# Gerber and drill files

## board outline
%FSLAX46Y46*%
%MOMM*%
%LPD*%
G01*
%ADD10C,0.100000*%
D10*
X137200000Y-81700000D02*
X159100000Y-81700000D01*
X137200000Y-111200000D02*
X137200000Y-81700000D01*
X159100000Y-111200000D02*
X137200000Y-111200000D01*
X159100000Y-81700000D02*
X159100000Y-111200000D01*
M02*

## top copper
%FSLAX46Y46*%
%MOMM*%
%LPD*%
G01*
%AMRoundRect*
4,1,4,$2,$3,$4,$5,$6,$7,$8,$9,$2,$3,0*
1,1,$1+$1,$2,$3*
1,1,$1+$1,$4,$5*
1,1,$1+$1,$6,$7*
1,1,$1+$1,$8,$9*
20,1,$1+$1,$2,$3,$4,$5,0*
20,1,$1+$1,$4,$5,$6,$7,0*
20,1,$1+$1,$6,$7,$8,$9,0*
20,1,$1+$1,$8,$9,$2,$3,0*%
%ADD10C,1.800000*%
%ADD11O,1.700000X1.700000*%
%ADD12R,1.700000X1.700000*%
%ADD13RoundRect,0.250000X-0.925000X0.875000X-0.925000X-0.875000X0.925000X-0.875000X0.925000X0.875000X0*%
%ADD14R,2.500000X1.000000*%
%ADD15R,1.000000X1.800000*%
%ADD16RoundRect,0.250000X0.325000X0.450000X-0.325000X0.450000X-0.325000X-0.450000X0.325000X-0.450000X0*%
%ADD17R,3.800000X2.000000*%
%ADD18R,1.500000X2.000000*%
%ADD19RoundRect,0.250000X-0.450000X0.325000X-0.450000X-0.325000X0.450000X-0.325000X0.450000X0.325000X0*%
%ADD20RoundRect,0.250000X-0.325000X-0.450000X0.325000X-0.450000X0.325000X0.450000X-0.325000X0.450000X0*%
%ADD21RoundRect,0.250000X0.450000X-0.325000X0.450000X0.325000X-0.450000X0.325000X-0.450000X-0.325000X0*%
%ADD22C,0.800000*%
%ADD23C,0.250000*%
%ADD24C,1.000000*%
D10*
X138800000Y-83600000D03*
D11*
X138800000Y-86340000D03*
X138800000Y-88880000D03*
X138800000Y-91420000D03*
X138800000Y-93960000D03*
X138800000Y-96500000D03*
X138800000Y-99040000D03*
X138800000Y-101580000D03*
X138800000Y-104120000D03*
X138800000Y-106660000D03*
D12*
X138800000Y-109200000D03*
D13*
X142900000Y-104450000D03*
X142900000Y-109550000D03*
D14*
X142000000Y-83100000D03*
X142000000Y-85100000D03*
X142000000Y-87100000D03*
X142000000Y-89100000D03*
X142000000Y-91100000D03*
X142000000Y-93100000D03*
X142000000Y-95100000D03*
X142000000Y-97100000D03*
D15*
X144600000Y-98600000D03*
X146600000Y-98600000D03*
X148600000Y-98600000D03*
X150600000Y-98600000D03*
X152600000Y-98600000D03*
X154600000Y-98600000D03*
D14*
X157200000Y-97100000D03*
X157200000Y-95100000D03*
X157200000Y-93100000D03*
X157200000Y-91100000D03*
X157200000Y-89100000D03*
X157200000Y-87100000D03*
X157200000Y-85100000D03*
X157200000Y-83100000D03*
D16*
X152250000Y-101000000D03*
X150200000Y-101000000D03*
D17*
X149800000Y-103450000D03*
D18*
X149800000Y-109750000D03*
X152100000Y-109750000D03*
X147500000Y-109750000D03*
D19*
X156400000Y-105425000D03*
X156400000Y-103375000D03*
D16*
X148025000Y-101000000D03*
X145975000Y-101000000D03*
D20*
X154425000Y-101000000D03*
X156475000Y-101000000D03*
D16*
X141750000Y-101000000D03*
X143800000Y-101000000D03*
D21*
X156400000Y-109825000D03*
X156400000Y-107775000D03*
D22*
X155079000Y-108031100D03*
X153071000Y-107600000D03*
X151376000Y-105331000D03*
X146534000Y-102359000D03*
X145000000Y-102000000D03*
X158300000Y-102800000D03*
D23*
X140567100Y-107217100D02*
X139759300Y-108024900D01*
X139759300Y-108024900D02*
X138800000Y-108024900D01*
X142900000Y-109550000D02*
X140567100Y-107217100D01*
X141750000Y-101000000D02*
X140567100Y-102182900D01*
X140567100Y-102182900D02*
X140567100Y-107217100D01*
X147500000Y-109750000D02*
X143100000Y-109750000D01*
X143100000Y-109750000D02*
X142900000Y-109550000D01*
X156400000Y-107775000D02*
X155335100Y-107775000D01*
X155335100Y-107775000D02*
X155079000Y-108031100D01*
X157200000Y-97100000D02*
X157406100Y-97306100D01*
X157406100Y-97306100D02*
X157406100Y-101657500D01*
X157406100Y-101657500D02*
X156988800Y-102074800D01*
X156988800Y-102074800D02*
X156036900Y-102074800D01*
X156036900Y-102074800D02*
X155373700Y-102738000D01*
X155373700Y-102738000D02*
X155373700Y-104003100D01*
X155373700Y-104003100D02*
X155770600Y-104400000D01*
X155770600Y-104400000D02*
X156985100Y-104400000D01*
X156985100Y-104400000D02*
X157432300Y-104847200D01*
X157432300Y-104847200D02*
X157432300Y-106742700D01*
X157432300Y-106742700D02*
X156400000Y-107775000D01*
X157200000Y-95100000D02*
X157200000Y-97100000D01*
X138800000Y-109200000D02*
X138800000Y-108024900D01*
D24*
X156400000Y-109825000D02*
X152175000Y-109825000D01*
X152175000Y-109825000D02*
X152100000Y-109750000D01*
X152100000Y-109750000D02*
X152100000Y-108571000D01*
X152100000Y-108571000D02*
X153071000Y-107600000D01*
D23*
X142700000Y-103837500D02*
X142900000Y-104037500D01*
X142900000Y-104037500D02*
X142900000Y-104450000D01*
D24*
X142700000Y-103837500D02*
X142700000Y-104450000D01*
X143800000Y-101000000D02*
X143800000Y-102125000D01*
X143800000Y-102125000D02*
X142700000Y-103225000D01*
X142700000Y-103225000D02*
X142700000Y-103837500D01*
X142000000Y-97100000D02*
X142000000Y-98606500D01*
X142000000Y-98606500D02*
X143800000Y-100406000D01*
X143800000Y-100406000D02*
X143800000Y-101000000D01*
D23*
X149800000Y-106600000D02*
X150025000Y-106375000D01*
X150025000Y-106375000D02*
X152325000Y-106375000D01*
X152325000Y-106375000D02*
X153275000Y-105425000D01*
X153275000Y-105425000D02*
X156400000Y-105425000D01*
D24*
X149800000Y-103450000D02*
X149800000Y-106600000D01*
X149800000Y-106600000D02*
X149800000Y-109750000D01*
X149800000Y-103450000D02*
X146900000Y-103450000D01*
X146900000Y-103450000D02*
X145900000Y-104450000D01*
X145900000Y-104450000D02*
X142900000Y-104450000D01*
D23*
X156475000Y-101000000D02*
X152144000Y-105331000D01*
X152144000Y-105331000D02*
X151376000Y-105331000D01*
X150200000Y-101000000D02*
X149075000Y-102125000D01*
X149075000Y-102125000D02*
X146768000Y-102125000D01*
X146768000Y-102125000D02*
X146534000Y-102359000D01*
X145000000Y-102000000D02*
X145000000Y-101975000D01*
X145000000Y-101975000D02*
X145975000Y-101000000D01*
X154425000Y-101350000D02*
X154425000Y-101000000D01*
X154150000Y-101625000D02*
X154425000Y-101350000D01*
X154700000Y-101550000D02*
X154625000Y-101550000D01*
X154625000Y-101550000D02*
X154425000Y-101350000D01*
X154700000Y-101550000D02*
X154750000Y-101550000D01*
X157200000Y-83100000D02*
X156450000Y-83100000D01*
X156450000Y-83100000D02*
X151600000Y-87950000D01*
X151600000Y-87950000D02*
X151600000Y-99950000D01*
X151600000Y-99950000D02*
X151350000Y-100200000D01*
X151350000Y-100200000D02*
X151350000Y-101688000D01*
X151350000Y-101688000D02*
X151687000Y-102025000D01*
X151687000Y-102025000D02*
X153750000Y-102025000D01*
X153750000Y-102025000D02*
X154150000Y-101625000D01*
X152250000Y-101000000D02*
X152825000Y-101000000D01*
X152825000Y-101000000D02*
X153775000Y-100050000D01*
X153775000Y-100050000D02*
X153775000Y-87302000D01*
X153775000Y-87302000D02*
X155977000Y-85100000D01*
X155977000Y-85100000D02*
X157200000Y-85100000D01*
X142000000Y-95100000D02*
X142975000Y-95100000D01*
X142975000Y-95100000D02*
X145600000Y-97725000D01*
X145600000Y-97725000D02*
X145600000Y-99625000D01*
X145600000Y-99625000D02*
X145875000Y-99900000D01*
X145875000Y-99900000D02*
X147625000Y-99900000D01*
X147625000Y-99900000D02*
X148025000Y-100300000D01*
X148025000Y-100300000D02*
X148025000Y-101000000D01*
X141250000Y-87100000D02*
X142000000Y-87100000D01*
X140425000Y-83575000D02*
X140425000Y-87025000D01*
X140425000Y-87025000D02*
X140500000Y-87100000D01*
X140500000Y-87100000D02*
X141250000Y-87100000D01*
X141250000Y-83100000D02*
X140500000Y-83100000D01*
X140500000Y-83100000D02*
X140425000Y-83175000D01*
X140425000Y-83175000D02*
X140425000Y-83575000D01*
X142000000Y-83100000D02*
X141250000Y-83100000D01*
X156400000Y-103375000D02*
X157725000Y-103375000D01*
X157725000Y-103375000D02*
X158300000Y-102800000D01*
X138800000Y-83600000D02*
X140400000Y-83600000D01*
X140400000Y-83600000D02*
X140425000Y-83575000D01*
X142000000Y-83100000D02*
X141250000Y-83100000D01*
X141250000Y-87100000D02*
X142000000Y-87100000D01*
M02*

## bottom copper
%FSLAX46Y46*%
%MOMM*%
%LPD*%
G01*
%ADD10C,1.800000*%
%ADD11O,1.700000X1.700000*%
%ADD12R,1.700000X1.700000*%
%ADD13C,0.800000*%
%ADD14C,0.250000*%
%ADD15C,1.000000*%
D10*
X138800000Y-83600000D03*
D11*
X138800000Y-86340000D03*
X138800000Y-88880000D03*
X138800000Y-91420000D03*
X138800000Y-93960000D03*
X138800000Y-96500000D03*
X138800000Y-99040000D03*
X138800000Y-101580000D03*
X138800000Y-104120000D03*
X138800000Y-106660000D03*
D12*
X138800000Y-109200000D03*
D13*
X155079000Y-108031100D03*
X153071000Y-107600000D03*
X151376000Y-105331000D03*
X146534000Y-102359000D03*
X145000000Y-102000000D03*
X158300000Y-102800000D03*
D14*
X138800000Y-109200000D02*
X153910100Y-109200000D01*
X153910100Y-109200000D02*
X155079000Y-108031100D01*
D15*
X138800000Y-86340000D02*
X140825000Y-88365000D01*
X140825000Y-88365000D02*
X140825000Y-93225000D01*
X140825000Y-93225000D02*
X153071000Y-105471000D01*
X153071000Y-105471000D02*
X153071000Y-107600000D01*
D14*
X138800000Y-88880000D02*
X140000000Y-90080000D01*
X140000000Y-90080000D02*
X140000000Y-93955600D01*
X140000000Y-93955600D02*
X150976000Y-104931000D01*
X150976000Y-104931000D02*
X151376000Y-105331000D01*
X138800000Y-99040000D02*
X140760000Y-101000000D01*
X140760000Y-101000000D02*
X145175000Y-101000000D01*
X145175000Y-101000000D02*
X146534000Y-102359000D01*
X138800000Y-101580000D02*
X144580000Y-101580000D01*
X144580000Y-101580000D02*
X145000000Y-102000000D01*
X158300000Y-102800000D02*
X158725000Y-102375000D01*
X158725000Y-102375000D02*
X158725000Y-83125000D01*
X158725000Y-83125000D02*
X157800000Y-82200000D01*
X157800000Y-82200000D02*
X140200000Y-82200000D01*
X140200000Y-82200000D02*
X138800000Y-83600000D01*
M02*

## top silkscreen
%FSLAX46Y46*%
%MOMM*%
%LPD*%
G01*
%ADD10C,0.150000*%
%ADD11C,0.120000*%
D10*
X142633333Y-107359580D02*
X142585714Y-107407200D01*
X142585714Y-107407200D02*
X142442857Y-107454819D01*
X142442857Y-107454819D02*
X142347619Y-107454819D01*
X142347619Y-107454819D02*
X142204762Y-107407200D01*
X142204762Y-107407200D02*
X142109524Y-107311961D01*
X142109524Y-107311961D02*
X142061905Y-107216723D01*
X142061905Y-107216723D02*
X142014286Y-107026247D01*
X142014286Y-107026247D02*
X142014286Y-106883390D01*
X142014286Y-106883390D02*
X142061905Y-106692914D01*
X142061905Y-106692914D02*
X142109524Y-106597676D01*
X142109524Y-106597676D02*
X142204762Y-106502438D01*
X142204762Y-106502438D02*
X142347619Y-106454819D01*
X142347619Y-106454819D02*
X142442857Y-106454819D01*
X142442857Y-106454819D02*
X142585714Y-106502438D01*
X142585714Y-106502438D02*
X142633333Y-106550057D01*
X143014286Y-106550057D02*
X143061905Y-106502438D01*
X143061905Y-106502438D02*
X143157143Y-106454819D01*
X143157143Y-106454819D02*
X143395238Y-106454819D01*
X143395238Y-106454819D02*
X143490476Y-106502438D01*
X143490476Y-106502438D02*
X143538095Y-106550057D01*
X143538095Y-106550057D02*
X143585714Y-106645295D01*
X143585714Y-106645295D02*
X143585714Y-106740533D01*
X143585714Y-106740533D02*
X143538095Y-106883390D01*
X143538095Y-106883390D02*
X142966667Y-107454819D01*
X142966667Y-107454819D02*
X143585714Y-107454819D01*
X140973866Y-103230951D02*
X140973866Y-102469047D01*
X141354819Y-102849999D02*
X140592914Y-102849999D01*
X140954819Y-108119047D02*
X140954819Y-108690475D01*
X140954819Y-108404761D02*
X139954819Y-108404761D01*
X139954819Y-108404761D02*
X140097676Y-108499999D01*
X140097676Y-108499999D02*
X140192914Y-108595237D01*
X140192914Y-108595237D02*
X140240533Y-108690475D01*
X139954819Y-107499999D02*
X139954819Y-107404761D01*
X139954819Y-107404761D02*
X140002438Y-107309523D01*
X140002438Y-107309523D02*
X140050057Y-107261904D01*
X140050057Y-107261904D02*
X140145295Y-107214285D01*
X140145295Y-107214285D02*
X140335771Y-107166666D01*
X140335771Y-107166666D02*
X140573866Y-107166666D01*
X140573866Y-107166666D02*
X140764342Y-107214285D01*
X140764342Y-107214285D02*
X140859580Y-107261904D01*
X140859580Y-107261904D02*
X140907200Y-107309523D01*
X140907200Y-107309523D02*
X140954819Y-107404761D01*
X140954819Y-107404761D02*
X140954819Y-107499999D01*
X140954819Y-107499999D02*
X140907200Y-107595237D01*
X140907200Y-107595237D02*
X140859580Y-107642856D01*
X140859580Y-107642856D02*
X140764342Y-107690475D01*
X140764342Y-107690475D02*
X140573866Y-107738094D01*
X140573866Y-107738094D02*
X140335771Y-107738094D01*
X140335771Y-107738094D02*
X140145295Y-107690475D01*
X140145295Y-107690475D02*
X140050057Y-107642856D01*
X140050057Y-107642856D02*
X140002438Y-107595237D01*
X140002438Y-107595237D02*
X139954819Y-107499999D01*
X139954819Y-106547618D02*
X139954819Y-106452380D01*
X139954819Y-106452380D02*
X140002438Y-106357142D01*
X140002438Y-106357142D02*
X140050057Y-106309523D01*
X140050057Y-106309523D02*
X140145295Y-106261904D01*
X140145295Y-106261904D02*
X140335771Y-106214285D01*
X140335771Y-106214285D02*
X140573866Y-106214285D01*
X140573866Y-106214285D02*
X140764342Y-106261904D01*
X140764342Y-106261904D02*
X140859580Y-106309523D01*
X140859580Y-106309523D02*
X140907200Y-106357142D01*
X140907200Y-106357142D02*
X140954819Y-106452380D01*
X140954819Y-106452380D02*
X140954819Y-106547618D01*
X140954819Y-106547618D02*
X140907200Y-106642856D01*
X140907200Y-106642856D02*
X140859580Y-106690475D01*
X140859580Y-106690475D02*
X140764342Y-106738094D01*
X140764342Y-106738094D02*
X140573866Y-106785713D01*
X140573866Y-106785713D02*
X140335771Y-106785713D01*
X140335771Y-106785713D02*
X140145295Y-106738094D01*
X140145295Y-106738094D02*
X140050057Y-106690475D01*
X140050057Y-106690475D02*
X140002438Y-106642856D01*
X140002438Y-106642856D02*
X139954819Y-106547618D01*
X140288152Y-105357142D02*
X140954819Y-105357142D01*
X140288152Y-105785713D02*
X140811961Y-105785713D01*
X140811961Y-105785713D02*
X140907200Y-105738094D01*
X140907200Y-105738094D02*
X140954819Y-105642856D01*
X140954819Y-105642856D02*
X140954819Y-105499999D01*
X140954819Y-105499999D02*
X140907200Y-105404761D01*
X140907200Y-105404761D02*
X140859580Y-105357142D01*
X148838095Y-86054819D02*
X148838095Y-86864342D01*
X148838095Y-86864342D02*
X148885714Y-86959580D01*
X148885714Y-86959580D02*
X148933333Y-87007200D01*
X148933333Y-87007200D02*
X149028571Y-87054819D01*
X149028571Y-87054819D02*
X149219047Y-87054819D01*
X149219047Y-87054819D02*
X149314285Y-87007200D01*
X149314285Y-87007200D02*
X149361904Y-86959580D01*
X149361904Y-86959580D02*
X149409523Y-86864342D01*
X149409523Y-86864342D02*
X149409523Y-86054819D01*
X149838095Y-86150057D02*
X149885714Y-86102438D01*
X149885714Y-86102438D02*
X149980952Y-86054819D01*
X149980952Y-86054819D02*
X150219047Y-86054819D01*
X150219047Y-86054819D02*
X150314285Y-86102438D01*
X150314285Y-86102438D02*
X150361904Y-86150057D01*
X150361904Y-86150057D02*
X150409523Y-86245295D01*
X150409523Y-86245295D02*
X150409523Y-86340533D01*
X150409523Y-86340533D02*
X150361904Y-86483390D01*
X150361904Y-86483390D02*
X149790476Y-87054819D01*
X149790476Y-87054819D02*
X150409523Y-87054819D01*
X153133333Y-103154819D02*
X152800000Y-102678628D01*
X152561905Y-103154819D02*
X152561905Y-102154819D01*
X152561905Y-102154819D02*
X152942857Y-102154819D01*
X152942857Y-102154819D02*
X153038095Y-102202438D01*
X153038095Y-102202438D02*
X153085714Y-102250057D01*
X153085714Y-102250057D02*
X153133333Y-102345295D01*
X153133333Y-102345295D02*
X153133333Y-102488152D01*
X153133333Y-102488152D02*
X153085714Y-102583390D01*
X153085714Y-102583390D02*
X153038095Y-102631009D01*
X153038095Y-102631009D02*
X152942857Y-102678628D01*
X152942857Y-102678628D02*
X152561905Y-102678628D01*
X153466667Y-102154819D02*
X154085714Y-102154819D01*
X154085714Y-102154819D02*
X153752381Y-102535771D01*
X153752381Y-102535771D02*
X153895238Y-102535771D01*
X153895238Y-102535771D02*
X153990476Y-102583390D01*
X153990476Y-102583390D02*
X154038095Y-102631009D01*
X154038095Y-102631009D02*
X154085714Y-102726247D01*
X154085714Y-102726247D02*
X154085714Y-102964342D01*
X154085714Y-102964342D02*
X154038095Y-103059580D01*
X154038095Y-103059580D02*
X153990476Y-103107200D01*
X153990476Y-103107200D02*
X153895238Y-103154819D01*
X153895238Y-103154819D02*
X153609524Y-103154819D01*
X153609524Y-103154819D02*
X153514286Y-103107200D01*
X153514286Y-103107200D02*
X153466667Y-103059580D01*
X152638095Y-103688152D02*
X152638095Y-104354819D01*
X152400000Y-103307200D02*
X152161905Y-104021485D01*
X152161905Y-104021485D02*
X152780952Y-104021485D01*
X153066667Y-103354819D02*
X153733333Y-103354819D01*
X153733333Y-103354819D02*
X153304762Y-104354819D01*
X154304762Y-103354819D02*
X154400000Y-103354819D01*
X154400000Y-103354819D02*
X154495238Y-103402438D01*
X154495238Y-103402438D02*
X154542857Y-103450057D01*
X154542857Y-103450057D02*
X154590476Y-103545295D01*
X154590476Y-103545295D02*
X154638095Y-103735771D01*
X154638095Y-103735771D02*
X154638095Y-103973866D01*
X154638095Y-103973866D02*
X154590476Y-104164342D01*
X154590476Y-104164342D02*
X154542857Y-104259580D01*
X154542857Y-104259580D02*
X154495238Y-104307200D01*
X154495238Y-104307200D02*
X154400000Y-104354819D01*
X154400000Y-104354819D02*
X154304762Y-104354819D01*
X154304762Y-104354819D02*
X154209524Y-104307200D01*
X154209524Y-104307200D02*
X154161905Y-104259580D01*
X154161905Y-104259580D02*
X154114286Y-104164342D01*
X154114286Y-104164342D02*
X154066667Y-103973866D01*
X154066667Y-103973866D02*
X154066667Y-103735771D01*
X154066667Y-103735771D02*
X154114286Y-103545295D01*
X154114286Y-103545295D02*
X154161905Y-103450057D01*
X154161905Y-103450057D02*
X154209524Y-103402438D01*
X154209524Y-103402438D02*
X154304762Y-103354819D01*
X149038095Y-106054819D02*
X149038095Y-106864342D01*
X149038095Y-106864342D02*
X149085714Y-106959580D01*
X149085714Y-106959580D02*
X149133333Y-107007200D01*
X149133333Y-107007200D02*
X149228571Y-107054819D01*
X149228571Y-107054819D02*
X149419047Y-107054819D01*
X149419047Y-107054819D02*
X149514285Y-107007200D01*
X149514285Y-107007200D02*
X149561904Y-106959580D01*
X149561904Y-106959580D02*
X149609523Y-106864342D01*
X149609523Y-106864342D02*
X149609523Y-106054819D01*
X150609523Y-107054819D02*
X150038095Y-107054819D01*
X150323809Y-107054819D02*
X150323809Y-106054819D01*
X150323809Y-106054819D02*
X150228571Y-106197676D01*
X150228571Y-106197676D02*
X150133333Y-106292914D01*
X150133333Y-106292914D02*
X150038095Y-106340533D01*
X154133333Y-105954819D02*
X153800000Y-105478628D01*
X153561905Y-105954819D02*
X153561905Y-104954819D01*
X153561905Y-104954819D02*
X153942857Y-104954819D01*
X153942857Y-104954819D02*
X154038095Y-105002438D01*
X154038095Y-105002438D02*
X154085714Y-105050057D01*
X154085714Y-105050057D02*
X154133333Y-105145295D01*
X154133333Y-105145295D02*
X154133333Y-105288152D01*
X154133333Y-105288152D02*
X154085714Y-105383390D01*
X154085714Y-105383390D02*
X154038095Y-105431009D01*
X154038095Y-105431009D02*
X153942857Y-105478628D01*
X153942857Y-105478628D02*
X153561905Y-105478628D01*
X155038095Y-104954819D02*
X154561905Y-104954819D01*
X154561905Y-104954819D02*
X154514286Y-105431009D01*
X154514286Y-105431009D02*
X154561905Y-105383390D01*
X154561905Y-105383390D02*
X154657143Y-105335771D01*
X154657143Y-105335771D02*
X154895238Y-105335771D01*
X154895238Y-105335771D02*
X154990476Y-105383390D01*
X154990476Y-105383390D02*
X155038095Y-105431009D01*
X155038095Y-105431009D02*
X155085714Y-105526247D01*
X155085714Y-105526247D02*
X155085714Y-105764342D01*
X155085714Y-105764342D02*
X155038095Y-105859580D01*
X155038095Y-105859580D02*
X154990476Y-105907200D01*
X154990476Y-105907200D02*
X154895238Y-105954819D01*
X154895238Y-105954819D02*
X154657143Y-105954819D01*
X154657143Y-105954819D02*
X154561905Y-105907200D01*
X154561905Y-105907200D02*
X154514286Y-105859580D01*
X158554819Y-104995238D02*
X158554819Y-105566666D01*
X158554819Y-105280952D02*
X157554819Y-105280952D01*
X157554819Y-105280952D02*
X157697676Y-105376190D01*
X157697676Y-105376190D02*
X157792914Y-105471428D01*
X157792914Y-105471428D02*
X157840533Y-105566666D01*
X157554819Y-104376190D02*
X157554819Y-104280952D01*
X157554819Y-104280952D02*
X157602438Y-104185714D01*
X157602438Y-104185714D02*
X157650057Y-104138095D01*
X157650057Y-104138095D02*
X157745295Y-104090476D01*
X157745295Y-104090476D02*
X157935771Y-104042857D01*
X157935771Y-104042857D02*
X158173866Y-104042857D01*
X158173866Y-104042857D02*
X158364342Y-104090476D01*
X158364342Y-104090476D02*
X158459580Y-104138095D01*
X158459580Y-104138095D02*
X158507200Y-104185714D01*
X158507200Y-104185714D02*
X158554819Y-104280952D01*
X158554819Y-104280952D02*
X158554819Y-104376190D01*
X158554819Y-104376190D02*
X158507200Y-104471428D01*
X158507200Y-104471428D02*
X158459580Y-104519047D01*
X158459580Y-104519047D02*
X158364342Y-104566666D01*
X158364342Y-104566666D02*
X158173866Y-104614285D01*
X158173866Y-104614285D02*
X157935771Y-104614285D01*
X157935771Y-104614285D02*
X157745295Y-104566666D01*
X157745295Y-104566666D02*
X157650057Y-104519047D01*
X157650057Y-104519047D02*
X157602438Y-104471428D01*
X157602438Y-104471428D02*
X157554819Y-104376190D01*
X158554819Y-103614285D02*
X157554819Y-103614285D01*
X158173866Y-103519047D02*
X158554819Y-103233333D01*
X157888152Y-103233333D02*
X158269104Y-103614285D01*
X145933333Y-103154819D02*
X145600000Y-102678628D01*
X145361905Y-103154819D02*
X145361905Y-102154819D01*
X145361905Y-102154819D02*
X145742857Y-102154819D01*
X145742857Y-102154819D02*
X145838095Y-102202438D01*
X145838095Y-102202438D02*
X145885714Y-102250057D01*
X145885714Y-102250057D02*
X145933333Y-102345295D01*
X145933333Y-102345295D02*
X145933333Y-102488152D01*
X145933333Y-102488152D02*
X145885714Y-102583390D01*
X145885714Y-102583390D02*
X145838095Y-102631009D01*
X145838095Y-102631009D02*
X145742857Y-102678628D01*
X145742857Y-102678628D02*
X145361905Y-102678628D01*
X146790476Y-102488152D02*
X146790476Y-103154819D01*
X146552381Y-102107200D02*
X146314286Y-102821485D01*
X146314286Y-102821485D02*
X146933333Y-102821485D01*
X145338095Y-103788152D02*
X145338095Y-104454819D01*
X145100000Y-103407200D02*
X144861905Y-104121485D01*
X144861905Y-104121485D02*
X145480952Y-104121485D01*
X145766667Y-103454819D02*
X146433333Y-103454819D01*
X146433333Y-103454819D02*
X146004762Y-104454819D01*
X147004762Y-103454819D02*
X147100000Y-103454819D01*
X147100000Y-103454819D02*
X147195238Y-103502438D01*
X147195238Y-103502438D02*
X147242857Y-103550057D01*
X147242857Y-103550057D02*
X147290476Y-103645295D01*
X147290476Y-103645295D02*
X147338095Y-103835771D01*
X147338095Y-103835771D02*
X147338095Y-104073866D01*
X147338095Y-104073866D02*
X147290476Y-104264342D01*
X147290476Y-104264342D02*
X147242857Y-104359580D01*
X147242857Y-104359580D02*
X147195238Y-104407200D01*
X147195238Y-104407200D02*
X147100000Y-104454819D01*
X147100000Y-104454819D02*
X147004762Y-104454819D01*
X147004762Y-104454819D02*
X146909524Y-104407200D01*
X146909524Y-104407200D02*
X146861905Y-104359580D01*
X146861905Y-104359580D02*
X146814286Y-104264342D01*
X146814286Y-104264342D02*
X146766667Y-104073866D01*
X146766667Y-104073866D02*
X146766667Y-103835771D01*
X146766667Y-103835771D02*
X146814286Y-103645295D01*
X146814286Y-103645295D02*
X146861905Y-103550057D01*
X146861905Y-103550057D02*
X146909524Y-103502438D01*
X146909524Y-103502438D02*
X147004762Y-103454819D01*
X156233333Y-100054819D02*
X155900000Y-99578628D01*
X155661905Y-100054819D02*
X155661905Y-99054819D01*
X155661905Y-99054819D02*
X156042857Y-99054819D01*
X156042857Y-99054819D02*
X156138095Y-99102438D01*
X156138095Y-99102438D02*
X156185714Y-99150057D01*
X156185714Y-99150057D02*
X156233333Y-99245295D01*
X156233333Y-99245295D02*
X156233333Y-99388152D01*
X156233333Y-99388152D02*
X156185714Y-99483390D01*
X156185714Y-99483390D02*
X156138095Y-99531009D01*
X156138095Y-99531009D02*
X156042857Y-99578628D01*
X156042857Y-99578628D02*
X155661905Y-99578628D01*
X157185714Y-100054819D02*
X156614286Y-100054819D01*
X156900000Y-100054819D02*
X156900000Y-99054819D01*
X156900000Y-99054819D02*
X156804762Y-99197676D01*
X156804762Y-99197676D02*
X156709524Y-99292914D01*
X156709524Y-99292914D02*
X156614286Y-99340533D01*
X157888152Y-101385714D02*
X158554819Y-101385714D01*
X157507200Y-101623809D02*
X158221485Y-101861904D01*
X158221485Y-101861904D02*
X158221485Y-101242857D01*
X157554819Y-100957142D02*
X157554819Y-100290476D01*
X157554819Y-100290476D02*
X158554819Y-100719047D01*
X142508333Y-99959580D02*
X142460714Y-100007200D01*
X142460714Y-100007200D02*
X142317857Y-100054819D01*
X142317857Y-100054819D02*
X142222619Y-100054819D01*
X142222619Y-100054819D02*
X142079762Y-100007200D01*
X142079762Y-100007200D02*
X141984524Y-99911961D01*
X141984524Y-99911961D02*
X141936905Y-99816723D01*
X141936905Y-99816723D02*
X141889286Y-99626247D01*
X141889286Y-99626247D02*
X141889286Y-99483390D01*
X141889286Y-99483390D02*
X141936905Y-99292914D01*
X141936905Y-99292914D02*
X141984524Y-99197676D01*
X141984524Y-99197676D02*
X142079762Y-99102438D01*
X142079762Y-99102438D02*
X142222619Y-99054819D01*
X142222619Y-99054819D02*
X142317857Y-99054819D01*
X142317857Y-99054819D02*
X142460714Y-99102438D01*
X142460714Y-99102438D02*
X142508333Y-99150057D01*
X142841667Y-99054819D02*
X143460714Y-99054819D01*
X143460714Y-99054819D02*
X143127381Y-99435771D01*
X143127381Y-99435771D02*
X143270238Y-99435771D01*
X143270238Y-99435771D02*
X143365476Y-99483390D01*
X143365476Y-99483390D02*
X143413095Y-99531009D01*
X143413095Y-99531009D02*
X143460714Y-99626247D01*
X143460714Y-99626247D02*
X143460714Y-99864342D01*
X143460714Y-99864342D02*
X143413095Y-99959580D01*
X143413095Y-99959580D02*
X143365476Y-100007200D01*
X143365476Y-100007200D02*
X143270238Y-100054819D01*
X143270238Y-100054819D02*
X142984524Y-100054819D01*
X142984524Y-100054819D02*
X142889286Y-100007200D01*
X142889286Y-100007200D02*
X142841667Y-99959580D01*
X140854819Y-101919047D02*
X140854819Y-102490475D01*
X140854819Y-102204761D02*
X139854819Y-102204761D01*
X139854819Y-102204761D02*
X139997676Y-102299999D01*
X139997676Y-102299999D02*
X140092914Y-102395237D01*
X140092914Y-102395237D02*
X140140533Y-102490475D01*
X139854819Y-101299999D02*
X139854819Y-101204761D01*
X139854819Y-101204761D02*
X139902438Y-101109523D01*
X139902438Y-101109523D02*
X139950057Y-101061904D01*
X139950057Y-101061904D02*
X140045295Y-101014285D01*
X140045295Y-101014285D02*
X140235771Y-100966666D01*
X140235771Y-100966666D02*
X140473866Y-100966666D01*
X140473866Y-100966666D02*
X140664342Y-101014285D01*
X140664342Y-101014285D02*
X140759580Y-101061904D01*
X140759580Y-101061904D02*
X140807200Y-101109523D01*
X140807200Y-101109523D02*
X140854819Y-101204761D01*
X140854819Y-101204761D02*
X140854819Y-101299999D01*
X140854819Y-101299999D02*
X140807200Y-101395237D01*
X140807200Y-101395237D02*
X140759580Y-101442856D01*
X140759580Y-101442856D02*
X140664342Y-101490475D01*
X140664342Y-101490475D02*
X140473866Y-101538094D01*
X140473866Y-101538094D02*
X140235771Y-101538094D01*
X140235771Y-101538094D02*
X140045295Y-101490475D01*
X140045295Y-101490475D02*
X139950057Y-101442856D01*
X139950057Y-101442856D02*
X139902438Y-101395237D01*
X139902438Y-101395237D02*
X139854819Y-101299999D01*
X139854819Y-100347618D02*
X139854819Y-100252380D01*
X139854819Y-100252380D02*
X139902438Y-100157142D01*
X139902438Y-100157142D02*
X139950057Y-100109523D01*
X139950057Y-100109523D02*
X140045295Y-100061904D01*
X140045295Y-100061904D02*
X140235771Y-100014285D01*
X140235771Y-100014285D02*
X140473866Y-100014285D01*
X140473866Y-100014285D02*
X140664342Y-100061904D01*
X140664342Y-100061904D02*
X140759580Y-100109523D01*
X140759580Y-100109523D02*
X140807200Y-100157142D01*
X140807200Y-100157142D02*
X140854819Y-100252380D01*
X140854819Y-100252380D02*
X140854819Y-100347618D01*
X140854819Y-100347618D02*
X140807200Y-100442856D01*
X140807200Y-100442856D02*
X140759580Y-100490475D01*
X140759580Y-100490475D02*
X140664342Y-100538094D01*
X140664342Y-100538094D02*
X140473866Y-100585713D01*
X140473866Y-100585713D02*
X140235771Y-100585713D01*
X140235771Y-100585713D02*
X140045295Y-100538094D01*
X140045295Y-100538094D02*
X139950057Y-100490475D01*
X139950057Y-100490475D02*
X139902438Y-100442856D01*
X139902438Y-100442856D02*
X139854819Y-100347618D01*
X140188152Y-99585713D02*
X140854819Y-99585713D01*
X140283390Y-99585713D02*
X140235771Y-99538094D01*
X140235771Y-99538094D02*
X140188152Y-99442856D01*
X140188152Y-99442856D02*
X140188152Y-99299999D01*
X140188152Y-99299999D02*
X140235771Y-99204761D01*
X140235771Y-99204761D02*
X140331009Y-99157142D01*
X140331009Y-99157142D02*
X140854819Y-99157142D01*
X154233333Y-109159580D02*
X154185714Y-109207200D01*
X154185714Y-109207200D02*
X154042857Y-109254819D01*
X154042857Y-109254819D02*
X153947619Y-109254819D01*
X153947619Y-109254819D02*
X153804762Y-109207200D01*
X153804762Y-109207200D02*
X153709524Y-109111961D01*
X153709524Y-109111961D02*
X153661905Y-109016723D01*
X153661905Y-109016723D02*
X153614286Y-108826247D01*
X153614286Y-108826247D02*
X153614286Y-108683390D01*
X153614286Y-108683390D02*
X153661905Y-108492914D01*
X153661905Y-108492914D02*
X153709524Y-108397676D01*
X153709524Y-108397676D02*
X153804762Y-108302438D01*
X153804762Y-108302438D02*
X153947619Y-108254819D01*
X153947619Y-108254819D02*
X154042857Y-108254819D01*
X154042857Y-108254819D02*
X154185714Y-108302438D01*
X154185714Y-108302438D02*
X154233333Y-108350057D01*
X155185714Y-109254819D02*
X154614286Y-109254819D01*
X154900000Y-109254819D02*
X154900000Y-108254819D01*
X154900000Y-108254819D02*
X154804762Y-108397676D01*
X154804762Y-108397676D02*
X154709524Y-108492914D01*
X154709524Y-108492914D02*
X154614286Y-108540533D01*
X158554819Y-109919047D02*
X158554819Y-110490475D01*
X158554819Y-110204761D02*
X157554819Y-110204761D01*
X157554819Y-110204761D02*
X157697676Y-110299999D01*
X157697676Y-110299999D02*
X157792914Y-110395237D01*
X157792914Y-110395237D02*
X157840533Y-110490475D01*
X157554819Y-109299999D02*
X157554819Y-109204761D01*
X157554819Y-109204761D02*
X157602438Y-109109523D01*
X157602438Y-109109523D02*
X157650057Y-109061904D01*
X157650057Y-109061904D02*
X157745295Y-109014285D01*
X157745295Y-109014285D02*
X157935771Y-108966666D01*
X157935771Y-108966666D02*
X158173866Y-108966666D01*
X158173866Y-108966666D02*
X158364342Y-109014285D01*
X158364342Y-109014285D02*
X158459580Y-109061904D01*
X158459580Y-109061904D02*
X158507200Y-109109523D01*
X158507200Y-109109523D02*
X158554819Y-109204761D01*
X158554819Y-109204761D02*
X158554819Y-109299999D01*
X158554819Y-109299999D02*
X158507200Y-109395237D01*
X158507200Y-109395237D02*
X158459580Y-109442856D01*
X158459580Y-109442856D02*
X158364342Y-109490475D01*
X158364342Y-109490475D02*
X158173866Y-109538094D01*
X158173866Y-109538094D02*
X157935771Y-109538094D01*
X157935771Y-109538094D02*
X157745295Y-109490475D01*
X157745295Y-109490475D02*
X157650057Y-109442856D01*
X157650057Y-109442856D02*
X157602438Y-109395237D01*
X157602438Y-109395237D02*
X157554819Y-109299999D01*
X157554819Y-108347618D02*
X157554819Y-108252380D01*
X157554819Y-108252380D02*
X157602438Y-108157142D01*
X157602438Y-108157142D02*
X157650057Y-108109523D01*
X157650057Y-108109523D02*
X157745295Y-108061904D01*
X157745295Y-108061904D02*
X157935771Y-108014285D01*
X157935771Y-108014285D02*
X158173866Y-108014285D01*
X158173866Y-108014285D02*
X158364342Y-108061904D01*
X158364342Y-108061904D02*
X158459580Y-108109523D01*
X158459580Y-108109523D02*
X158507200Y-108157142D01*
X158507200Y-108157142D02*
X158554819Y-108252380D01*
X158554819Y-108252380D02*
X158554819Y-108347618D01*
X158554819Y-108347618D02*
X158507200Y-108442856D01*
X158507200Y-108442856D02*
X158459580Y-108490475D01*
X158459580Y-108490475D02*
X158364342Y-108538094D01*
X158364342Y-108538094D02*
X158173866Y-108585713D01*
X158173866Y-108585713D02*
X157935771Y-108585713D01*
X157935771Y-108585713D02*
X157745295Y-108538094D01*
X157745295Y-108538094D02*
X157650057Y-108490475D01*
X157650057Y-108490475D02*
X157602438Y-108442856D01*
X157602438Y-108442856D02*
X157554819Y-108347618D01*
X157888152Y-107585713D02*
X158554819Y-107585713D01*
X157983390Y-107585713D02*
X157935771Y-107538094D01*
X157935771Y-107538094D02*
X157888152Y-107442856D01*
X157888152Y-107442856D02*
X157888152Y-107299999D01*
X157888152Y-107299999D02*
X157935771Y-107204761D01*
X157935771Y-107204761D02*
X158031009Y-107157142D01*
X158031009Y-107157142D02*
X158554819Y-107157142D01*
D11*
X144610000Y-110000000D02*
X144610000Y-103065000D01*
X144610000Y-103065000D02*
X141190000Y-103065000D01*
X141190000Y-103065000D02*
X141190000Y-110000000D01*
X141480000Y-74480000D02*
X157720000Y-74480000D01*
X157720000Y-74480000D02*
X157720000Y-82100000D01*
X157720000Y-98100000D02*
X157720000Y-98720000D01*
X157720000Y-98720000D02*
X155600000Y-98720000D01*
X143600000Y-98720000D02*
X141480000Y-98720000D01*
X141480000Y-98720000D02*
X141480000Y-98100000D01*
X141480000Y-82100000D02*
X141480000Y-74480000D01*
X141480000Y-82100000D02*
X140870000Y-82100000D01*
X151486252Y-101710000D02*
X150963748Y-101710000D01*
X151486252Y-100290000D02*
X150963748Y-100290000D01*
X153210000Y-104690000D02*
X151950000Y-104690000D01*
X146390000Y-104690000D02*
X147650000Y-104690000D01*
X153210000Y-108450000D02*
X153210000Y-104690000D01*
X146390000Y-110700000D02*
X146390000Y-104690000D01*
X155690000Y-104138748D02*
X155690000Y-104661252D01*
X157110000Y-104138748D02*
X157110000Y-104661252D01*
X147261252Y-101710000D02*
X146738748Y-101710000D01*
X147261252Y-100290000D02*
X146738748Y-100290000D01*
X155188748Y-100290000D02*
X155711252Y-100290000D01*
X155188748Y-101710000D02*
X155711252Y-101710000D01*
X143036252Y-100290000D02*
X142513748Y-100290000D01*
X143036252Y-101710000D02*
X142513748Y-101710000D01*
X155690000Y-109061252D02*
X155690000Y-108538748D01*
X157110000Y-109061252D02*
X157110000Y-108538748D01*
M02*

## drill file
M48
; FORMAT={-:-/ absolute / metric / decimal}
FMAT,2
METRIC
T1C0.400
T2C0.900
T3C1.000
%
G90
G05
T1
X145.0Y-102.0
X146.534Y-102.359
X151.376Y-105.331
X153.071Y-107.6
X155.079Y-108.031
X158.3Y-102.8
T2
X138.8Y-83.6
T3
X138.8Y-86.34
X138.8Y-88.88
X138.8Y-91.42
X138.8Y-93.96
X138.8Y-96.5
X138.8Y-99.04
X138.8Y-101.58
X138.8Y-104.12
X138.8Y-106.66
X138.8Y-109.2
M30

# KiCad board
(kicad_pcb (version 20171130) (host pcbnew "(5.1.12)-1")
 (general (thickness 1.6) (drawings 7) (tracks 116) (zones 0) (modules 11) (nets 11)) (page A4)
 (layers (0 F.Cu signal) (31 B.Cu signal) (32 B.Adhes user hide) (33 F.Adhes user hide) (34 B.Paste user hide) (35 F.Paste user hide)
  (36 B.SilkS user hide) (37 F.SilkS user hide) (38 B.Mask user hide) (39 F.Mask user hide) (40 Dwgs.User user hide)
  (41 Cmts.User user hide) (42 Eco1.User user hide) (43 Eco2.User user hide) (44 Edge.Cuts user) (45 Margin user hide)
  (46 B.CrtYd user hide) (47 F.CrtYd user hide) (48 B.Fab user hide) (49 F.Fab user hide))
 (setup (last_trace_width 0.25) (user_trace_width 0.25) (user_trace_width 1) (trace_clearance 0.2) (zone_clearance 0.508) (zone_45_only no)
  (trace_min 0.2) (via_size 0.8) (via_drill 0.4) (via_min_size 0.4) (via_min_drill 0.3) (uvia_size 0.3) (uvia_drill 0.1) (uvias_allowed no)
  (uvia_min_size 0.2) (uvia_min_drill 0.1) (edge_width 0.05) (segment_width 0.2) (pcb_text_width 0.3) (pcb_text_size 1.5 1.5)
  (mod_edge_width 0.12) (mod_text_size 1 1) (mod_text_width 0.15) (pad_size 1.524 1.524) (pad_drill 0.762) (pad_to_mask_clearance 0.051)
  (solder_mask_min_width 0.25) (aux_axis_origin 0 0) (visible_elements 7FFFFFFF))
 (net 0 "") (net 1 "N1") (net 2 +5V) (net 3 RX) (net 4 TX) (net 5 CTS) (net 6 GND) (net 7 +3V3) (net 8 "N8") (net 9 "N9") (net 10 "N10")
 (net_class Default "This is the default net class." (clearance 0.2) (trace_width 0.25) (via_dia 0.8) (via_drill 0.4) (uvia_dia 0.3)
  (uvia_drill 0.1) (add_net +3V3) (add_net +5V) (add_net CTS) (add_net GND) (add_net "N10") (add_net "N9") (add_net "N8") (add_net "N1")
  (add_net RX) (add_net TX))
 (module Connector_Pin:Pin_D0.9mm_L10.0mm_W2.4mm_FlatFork (layer B.Cu) (at 138.8 83.6)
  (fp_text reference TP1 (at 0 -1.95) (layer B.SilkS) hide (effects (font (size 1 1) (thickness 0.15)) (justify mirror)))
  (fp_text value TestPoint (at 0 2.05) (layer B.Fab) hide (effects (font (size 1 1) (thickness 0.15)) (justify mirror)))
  (pad 1 thru_hole circle (at 0 0) (size 1.8 1.8) (drill 0.9) (layers *.Cu *.Mask) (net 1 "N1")))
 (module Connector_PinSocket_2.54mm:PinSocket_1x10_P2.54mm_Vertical (layer B.Cu) (at 138.8 109.2)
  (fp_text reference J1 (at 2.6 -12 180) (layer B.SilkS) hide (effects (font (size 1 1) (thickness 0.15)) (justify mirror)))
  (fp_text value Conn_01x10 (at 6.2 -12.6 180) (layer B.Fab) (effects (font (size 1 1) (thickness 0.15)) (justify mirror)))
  (pad 10 thru_hole oval (at 0 -22.86) (size 1.7 1.7) (drill 1) (layers *.Cu *.Mask) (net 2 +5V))
  (pad 9 thru_hole oval (at 0 -20.32) (size 1.7 1.7) (drill 1) (layers *.Cu *.Mask) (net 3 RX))
  (pad 8 thru_hole oval (at 0 -17.78) (size 1.7 1.7) (drill 1) (layers *.Cu *.Mask))
  (pad 7 thru_hole oval (at 0 -15.24) (size 1.7 1.7) (drill 1) (layers *.Cu *.Mask))
  (pad 6 thru_hole oval (at 0 -12.7) (size 1.7 1.7) (drill 1) (layers *.Cu *.Mask))
  (pad 5 thru_hole oval (at 0 -10.16) (size 1.7 1.7) (drill 1) (layers *.Cu *.Mask) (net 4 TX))
  (pad 4 thru_hole oval (at 0 -7.62) (size 1.7 1.7) (drill 1) (layers *.Cu *.Mask) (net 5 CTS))
  (pad 3 thru_hole oval (at 0 -5.08) (size 1.7 1.7) (drill 1) (layers *.Cu *.Mask))
  (pad 2 thru_hole oval (at 0 -2.54) (size 1.7 1.7) (drill 1) (layers *.Cu *.Mask))
  (pad 1 thru_hole rect (at 0 0) (size 1.7 1.7) (drill 1) (layers *.Cu *.Mask) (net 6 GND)))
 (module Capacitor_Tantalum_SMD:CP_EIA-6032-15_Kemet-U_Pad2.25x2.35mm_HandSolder (layer F.Cu) (at 142.9 107 270)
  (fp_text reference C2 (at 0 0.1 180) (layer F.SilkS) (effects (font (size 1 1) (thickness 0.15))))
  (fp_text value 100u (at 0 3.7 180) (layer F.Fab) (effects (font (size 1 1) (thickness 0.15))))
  (fp_line (start 3 -1.71) (end -3.935 -1.71) (layer F.SilkS) (width 0.12))
  (fp_line (start -3.935 -1.71) (end -3.935 1.71) (layer F.SilkS) (width 0.12))
  (fp_line (start -3.935 1.71) (end 3 1.71) (layer F.SilkS) (width 0.12))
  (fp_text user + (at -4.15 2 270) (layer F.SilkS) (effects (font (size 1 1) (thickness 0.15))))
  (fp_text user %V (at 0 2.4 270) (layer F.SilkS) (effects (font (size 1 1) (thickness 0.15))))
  (pad 1 smd roundrect (at -2.55 0 270) (size 2.25 2.35) (layers F.Cu F.Paste F.Mask) (roundrect_rratio 0.111111) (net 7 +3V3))
  (pad 2 smd roundrect (at 2.55 0 270) (size 2.25 2.35) (layers F.Cu F.Paste F.Mask) (roundrect_rratio 0.111111) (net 6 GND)))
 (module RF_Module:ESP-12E (layer F.Cu) (at 149.6 86.6)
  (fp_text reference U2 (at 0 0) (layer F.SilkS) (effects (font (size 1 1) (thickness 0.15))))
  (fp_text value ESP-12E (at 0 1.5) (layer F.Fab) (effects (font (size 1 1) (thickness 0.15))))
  (fp_line (start -8.12 -12.12) (end 8.12 -12.12) (layer F.SilkS) (width 0.12))
  (fp_line (start 8.12 -12.12) (end 8.12 -4.5) (layer F.SilkS) (width 0.12))
  (fp_line (start 8.12 11.5) (end 8.12 12.12) (layer F.SilkS) (width 0.12))
  (fp_line (start 8.12 12.12) (end 6 12.12) (layer F.SilkS) (width 0.12))
  (fp_line (start -6 12.12) (end -8.12 12.12) (layer F.SilkS) (width 0.12))
  (fp_line (start -8.12 12.12) (end -8.12 11.5) (layer F.SilkS) (width 0.12))
  (fp_line (start -8.12 -4.5) (end -8.12 -12.12) (layer F.SilkS) (width 0.12))
  (fp_line (start -8.12 -4.5) (end -8.73 -4.5) (layer F.SilkS) (width 0.12))
  (pad 1 smd rect (at -7.6 -3.5) (size 2.5 1) (layers F.Cu F.Paste F.Mask) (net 1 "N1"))
  (pad 2 smd rect (at -7.6 -1.5) (size 2.5 1) (layers F.Cu F.Paste F.Mask))
  (pad 3 smd rect (at -7.6 0.5) (size 2.5 1) (layers F.Cu F.Paste F.Mask) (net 1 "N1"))
  (pad 4 smd rect (at -7.6 2.5) (size 2.5 1) (layers F.Cu F.Paste F.Mask))
  (pad 5 smd rect (at -7.6 4.5) (size 2.5 1) (layers F.Cu F.Paste F.Mask))
  (pad 6 smd rect (at -7.6 6.5) (size 2.5 1) (layers F.Cu F.Paste F.Mask))
  (pad 7 smd rect (at -7.6 8.5) (size 2.5 1) (layers F.Cu F.Paste F.Mask) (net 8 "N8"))
  (pad 8 smd rect (at -7.6 10.5) (size 2.5 1) (layers F.Cu F.Paste F.Mask) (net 7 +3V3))
  (pad 9 smd rect (at -5 12) (size 1 1.8) (layers F.Cu F.Paste F.Mask))
  (pad 10 smd rect (at -3 12) (size 1 1.8) (layers F.Cu F.Paste F.Mask))
  (pad 11 smd rect (at -1 12) (size 1 1.8) (layers F.Cu F.Paste F.Mask))
  (pad 12 smd rect (at 1 12) (size 1 1.8) (layers F.Cu F.Paste F.Mask))
  (pad 13 smd rect (at 3 12) (size 1 1.8) (layers F.Cu F.Paste F.Mask))
  (pad 14 smd rect (at 5 12) (size 1 1.8) (layers F.Cu F.Paste F.Mask))
  (pad 15 smd rect (at 7.6 10.5) (size 2.5 1) (layers F.Cu F.Paste F.Mask) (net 6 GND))
  (pad 16 smd rect (at 7.6 8.5) (size 2.5 1) (layers F.Cu F.Paste F.Mask) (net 6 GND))
  (pad 17 smd rect (at 7.6 6.5) (size 2.5 1) (layers F.Cu F.Paste F.Mask))
  (pad 18 smd rect (at 7.6 4.5) (size 2.5 1) (layers F.Cu F.Paste F.Mask))
  (pad 19 smd rect (at 7.6 2.5) (size 2.5 1) (layers F.Cu F.Paste F.Mask))
  (pad 20 smd rect (at 7.6 0.5) (size 2.5 1) (layers F.Cu F.Paste F.Mask))
  (pad 21 smd rect (at 7.6 -1.5) (size 2.5 1) (layers F.Cu F.Paste F.Mask) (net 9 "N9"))
  (pad 22 smd rect (at 7.6 -3.5) (size 2.5 1) (layers F.Cu F.Paste F.Mask) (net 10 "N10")))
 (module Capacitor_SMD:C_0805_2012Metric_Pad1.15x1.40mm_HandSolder (layer F.Cu) (at 151.225 101 180)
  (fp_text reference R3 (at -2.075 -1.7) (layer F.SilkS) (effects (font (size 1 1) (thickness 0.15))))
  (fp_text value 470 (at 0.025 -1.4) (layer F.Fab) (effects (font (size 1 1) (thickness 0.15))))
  (fp_line (start -0.261252 -0.71) (end 0.261252 -0.71) (layer F.SilkS) (width 0.12))
  (fp_line (start -0.261252 0.71) (end 0.261252 0.71) (layer F.SilkS) (width 0.12))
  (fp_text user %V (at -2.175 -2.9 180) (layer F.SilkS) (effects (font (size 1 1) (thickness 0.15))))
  (pad 1 smd roundrect (at -1.025 0 180) (size 1.15 1.4) (layers F.Cu F.Paste F.Mask) (roundrect_rratio 0.217391) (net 9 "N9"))
  (pad 2 smd roundrect (at 1.025 0 180) (size 1.15 1.4) (layers F.Cu F.Paste F.Mask) (roundrect_rratio 0.217391) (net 4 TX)))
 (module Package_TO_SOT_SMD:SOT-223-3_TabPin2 (layer F.Cu) (at 149.8 106.6 90)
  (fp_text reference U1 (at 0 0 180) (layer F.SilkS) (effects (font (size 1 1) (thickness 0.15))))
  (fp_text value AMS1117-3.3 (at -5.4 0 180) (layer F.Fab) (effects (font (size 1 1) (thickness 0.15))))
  (fp_line (start 1.91 3.41) (end 1.91 2.15) (layer F.SilkS) (width 0.12))
  (fp_line (start 1.91 -3.41) (end 1.91 -2.15) (layer F.SilkS) (width 0.12))
  (fp_line (start -1.85 3.41) (end 1.91 3.41) (layer F.SilkS) (width 0.12))
  (fp_line (start -4.1 -3.41) (end 1.91 -3.41) (layer F.SilkS) (width 0.12))
  (pad 2 smd rect (at 3.15 0 90) (size 2 3.8) (layers F.Cu F.Paste F.Mask) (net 7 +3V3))
  (pad 2 smd rect (at -3.15 0 90) (size 2 1.5) (layers F.Cu F.Paste F.Mask) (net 7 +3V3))
  (pad 3 smd rect (at -3.15 2.3 90) (size 2 1.5) (layers F.Cu F.Paste F.Mask) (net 2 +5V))
  (pad 1 smd rect (at -3.15 -2.3 90) (size 2 1.5) (layers F.Cu F.Paste F.Mask) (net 6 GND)))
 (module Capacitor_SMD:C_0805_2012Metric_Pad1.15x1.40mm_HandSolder (layer F.Cu) (at 156.4 104.4 270)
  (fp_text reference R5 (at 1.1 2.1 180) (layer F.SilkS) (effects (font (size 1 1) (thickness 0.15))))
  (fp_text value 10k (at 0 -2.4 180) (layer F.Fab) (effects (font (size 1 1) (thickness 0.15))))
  (fp_line (start -0.261252 0.71) (end 0.261252 0.71) (layer F.SilkS) (width 0.12))
  (fp_line (start -0.261252 -0.71) (end 0.261252 -0.71) (layer F.SilkS) (width 0.12))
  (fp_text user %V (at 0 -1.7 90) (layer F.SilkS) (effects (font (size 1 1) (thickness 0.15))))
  (pad 2 smd roundrect (at 1.025 0 270) (size 1.15 1.4) (layers F.Cu F.Paste F.Mask) (roundrect_rratio 0.217391) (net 7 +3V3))
  (pad 1 smd roundrect (at -1.025 0 270) (size 1.15 1.4) (layers F.Cu F.Paste F.Mask) (roundrect_rratio 0.217391) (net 1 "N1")))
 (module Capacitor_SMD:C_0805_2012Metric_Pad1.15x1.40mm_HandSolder (layer F.Cu) (at 147 101 180)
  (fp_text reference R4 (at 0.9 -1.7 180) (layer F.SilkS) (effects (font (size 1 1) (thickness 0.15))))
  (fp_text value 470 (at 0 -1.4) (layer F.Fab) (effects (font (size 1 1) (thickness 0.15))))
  (fp_line (start -0.261252 -0.71) (end 0.261252 -0.71) (layer F.SilkS) (width 0.12))
  (fp_line (start -0.261252 0.71) (end 0.261252 0.71) (layer F.SilkS) (width 0.12))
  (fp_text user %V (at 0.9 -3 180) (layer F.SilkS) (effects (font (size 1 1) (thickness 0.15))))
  (pad 1 smd roundrect (at -1.025 0 180) (size 1.15 1.4) (layers F.Cu F.Paste F.Mask) (roundrect_rratio 0.217391) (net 8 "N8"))
  (pad 2 smd roundrect (at 1.025 0 180) (size 1.15 1.4) (layers F.Cu F.Paste F.Mask) (roundrect_rratio 0.217391) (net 5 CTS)))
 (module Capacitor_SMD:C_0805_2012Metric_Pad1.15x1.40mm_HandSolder (layer F.Cu) (at 155.45 101)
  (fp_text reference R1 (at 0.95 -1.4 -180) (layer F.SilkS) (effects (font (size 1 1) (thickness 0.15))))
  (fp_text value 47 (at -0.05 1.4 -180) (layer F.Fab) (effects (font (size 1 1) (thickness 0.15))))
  (fp_line (start -0.261252 -0.71) (end 0.261252 -0.71) (layer F.SilkS) (width 0.12))
  (fp_line (start -0.261252 0.71) (end 0.261252 0.71) (layer F.SilkS) (width 0.12))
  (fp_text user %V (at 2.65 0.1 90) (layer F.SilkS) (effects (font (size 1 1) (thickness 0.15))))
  (pad 1 smd roundrect (at -1.025 0) (size 1.15 1.4) (layers F.Cu F.Paste F.Mask) (roundrect_rratio 0.217391) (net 10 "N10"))
  (pad 2 smd roundrect (at 1.025 0) (size 1.15 1.4) (layers F.Cu F.Paste F.Mask) (roundrect_rratio 0.217391) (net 3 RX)))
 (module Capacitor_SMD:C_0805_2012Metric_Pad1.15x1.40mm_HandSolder (layer F.Cu) (at 142.775 101 180)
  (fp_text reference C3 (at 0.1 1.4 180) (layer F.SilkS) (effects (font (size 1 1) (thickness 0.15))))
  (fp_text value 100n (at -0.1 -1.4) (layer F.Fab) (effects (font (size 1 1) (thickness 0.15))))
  (fp_line (start -0.261252 0.71) (end 0.261252 0.71) (layer F.SilkS) (width 0.12))
  (fp_line (start -0.261252 -0.71) (end 0.261252 -0.71) (layer F.SilkS) (width 0.12))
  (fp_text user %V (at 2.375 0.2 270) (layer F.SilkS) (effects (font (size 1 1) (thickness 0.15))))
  (pad 2 smd roundrect (at 1.025 0 180) (size 1.15 1.4) (layers F.Cu F.Paste F.Mask) (roundrect_rratio 0.217391) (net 6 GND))
  (pad 1 smd roundrect (at -1.025 0 180) (size 1.15 1.4) (layers F.Cu F.Paste F.Mask) (roundrect_rratio 0.217391) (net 7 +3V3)))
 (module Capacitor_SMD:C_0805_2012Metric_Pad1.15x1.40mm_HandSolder (layer F.Cu) (at 156.4 108.8 90)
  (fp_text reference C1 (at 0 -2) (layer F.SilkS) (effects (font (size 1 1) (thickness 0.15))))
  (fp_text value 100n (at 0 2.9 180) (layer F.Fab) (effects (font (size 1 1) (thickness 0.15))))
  (fp_line (start -0.261252 -0.71) (end 0.261252 -0.71) (layer F.SilkS) (width 0.12))
  (fp_line (start -0.261252 0.71) (end 0.261252 0.71) (layer F.SilkS) (width 0.12))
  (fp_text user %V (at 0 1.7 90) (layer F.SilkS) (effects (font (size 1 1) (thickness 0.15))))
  (pad 1 smd roundrect (at -1.025 0 90) (size 1.15 1.4) (layers F.Cu F.Paste F.Mask) (roundrect_rratio 0.217391) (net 2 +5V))
  (pad 2 smd roundrect (at 1.025 0 90) (size 1.15 1.4) (layers F.Cu F.Paste F.Mask) (roundrect_rratio 0.217391) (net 6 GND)))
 (gr_line (start 137.2 81.7) (end 159.1 81.7) (layer Edge.Cuts) (width 0.1))
 (gr_line (start 137.2 111.2) (end 137.2 81.7) (layer Edge.Cuts) (width 0.1))
 (gr_line (start 159.1 111.2) (end 137.2 111.2) (layer Edge.Cuts) (width 0.1))
 (gr_line (start 159.1 81.7) (end 159.1 111.2) (layer Edge.Cuts) (width 0.1))
 (segment (start 140.5671 107.2171) (end 139.7593 108.0249) (width 0.25) (layer F.Cu) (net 6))
 (segment (start 139.7593 108.0249) (end 138.8 108.0249) (width 0.25) (layer F.Cu) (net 6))
 (segment (start 142.9 109.55) (end 140.5671 107.2171) (width 0.25) (layer F.Cu) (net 6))
 (segment (start 141.75 101) (end 140.5671 102.1829) (width 0.25) (layer F.Cu) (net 6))
 (segment (start 140.5671 102.1829) (end 140.5671 107.2171) (width 0.25) (layer F.Cu) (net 6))
 (segment (start 147.5 109.75) (end 143.1 109.75) (width 0.25) (layer F.Cu) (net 6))
 (segment (start 143.1 109.75) (end 142.9 109.55) (width 0.25) (layer F.Cu) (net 6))
 (segment (start 156.4 107.775) (end 155.3351 107.775) (width 0.25) (layer F.Cu) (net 6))
 (segment (start 155.3351 107.775) (end 155.079 108.0311) (width 0.25) (layer F.Cu) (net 6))
 (segment (start 157.2 97.1) (end 157.4061 97.3061) (width 0.25) (layer F.Cu) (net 6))
 (segment (start 157.4061 97.3061) (end 157.4061 101.6575) (width 0.25) (layer F.Cu) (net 6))
 (segment (start 157.4061 101.6575) (end 156.9888 102.0748) (width 0.25) (layer F.Cu) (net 6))
 (segment (start 156.9888 102.0748) (end 156.0369 102.0748) (width 0.25) (layer F.Cu) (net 6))
 (segment (start 156.0369 102.0748) (end 155.3737 102.738) (width 0.25) (layer F.Cu) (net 6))
 (segment (start 155.3737 102.738) (end 155.3737 104.0031) (width 0.25) (layer F.Cu) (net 6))
 (segment (start 155.3737 104.0031) (end 155.7706 104.4) (width 0.25) (layer F.Cu) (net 6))
 (segment (start 155.7706 104.4) (end 156.9851 104.4) (width 0.25) (layer F.Cu) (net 6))
 (segment (start 156.9851 104.4) (end 157.4323 104.8472) (width 0.25) (layer F.Cu) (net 6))
 (segment (start 157.4323 104.8472) (end 157.4323 106.7427) (width 0.25) (layer F.Cu) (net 6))
 (segment (start 157.4323 106.7427) (end 156.4 107.775) (width 0.25) (layer F.Cu) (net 6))
 (segment (start 138.8 109.2) (end 153.9101 109.2) (width 0.25) (layer B.Cu) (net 6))
 (segment (start 153.9101 109.2) (end 155.079 108.0311) (width 0.25) (layer B.Cu) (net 6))
 (segment (start 157.2 95.1) (end 157.2 97.1) (width 0.25) (layer F.Cu) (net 6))
 (segment (start 138.8 109.2) (end 138.8 108.0249) (width 0.25) (layer F.Cu) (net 6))
 (via (at 155.079 108.0311) (size 0.8) (layers F.Cu B.Cu) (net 6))
 (segment (start 138.8 86.34) (end 140.825 88.365) (width 1) (layer B.Cu) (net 2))
 (segment (start 140.825 88.365) (end 140.825 93.225) (width 1) (layer B.Cu) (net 2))
 (segment (start 140.825 93.225) (end 153.071 105.471) (width 1) (layer B.Cu) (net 2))
 (segment (start 153.071 105.471) (end 153.071 107.6) (width 1) (layer B.Cu) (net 2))
 (segment (start 156.4 109.825) (end 152.175 109.825) (width 1) (layer F.Cu) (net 2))
 (segment (start 152.175 109.825) (end 152.1 109.75) (width 1) (layer F.Cu) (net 2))
 (segment (start 152.1 109.75) (end 152.1 108.571) (width 1) (layer F.Cu) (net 2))
 (segment (start 152.1 108.571) (end 153.071 107.6) (width 1) (layer F.Cu) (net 2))
 (via (at 153.071 107.6) (size 0.8) (layers F.Cu B.Cu) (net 2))
 (segment (start 142.7 103.8375) (end 142.9 104.0375) (width 0.25) (layer F.Cu) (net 7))
 (segment (start 142.9 104.0375) (end 142.9 104.45) (width 0.25) (layer F.Cu) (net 7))
 (segment (start 142.7 103.8375) (end 142.7 104.45) (width 1) (layer F.Cu) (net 7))
 (segment (start 143.8 101) (end 143.8 102.125) (width 1) (layer F.Cu) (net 7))
 (segment (start 143.8 102.125) (end 142.7 103.225) (width 1) (layer F.Cu) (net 7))
 (segment (start 142.7 103.225) (end 142.7 103.8375) (width 1) (layer F.Cu) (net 7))
 (segment (start 142 97.1) (end 142 98.6065) (width 1) (layer F.Cu) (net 7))
 (segment (start 142 98.6065) (end 143.8 100.406) (width 1) (layer F.Cu) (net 7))
 (segment (start 143.8 100.406) (end 143.8 101) (width 1) (layer F.Cu) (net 7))
 (segment (start 149.8 106.6) (end 150.025 106.375) (width 0.25) (layer F.Cu) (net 7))
 (segment (start 150.025 106.375) (end 152.325 106.375) (width 0.25) (layer F.Cu) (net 7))
 (segment (start 152.325 106.375) (end 153.275 105.425) (width 0.25) (layer F.Cu) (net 7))
 (segment (start 153.275 105.425) (end 156.4 105.425) (width 0.25) (layer F.Cu) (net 7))
 (segment (start 149.8 103.45) (end 149.8 106.6) (width 1) (layer F.Cu) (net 7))
 (segment (start 149.8 106.6) (end 149.8 109.75) (width 1) (layer F.Cu) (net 7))
 (segment (start 149.8 103.45) (end 146.9 103.45) (width 1) (layer F.Cu) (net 7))
 (segment (start 146.9 103.45) (end 145.9 104.45) (width 1) (layer F.Cu) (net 7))
 (segment (start 145.9 104.45) (end 142.9 104.45) (width 1) (layer F.Cu) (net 7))
 (segment (start 138.8 88.88) (end 140 90.08) (width 0.25) (layer B.Cu) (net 3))
 (segment (start 140 90.08) (end 140 93.9556) (width 0.25) (layer B.Cu) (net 3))
 (segment (start 140 93.9556) (end 150.976 104.931) (width 0.25) (layer B.Cu) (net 3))
 (segment (start 150.976 104.931) (end 151.376 105.331) (width 0.25) (layer B.Cu) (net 3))
 (segment (start 156.475 101) (end 152.144 105.331) (width 0.25) (layer F.Cu) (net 3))
 (segment (start 152.144 105.331) (end 151.376 105.331) (width 0.25) (layer F.Cu) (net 3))
 (via (at 151.376 105.331) (size 0.8) (layers F.Cu B.Cu) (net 3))
 (segment (start 138.8 99.04) (end 140.76 101) (width 0.25) (layer B.Cu) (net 4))
 (segment (start 140.76 101) (end 145.175 101) (width 0.25) (layer B.Cu) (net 4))
 (segment (start 145.175 101) (end 146.534 102.359) (width 0.25) (layer B.Cu) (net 4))
 (segment (start 150.2 101) (end 149.075 102.125) (width 0.25) (layer F.Cu) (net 4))
 (segment (start 149.075 102.125) (end 146.768 102.125) (width 0.25) (layer F.Cu) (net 4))
 (segment (start 146.768 102.125) (end 146.534 102.359) (width 0.25) (layer F.Cu) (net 4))
 (via (at 146.534 102.359) (size 0.8) (layers F.Cu B.Cu) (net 4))
 (segment (start 138.8 101.58) (end 144.58 101.58) (width 0.25) (layer B.Cu) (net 5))
 (segment (start 144.58 101.58) (end 145 102) (width 0.25) (layer B.Cu) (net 5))
 (segment (start 145 102) (end 145 101.975) (width 0.25) (layer F.Cu) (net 5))
 (segment (start 145 101.975) (end 145.975 101) (width 0.25) (layer F.Cu) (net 5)) (via (at 145 102) (size 0.8) (layers F.Cu B.Cu) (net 5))
 (segment (start 154.425 101.35) (end 154.425 101) (width 0.25) (layer F.Cu) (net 10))
 (segment (start 154.15 101.625) (end 154.425 101.35) (width 0.25) (layer F.Cu) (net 10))
 (segment (start 154.7 101.55) (end 154.625 101.55) (width 0.25) (layer F.Cu) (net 10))
 (segment (start 154.625 101.55) (end 154.425 101.35) (width 0.25) (layer F.Cu) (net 10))
 (segment (start 154.7 101.55) (end 154.75 101.55) (width 0.25) (layer F.Cu) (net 10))
 (segment (start 157.2 83.1) (end 156.45 83.1) (width 0.25) (layer F.Cu) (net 10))
 (segment (start 156.45 83.1) (end 151.6 87.95) (width 0.25) (layer F.Cu) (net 10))
 (segment (start 151.6 87.95) (end 151.6 99.95) (width 0.25) (layer F.Cu) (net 10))
 (segment (start 151.6 99.95) (end 151.35 100.2) (width 0.25) (layer F.Cu) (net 10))
 (segment (start 151.35 100.2) (end 151.35 101.688) (width 0.25) (layer F.Cu) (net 10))
 (segment (start 151.35 101.688) (end 151.687 102.025) (width 0.25) (layer F.Cu) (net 10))
 (segment (start 151.687 102.025) (end 153.75 102.025) (width 0.25) (layer F.Cu) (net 10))
 (segment (start 153.75 102.025) (end 154.15 101.625) (width 0.25) (layer F.Cu) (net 10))
 (segment (start 152.25 101) (end 152.825 101) (width 0.25) (layer F.Cu) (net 9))
 (segment (start 152.825 101) (end 153.775 100.05) (width 0.25) (layer F.Cu) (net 9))
 (segment (start 153.775 100.05) (end 153.775 87.302) (width 0.25) (layer F.Cu) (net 9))
 (segment (start 153.775 87.302) (end 155.977 85.1) (width 0.25) (layer F.Cu) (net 9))
 (segment (start 155.977 85.1) (end 157.2 85.1) (width 0.25) (layer F.Cu) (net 9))
 (segment (start 142 95.1) (end 142.975 95.1) (width 0.25) (layer F.Cu) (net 8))
 (segment (start 142.975 95.1) (end 145.6 97.725) (width 0.25) (layer F.Cu) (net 8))
 (segment (start 145.6 97.725) (end 145.6 99.625) (width 0.25) (layer F.Cu) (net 8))
 (segment (start 145.6 99.625) (end 145.875 99.9) (width 0.25) (layer F.Cu) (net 8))
 (segment (start 145.875 99.9) (end 147.625 99.9) (width 0.25) (layer F.Cu) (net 8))
 (segment (start 147.625 99.9) (end 148.025 100.3) (width 0.25) (layer F.Cu) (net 8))
 (segment (start 148.025 100.3) (end 148.025 101) (width 0.25) (layer F.Cu) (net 8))
 (segment (start 141.25 87.1) (end 142 87.1) (width 0.25) (layer F.Cu) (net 1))
 (segment (start 140.425 83.575) (end 140.425 87.025) (width 0.25) (layer F.Cu) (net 1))
 (segment (start 140.425 87.025) (end 140.5 87.1) (width 0.25) (layer F.Cu) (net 1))
 (segment (start 140.5 87.1) (end 141.25 87.1) (width 0.25) (layer F.Cu) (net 1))
 (segment (start 141.25 83.1) (end 140.5 83.1) (width 0.25) (layer F.Cu) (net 1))
 (segment (start 140.5 83.1) (end 140.425 83.175) (width 0.25) (layer F.Cu) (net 1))
 (segment (start 140.425 83.175) (end 140.425 83.575) (width 0.25) (layer F.Cu) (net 1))
 (segment (start 142 83.1) (end 141.25 83.1) (width 0.25) (layer F.Cu) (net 1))
 (segment (start 158.3 102.8) (end 158.725 102.375) (width 0.25) (layer B.Cu) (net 1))
 (segment (start 158.725 102.375) (end 158.725 83.125) (width 0.25) (layer B.Cu) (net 1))
 (segment (start 158.725 83.125) (end 157.8 82.2) (width 0.25) (layer B.Cu) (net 1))
 (segment (start 157.8 82.2) (end 140.2 82.2) (width 0.25) (layer B.Cu) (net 1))
 (segment (start 140.2 82.2) (end 138.8 83.6) (width 0.25) (layer B.Cu) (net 1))
 (segment (start 156.4 103.375) (end 157.725 103.375) (width 0.25) (layer F.Cu) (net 1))
 (segment (start 157.725 103.375) (end 158.3 102.8) (width 0.25) (layer F.Cu) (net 1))
 (segment (start 138.8 83.6) (end 140.4 83.6) (width 0.25) (layer F.Cu) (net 1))
 (segment (start 140.4 83.6) (end 140.425 83.575) (width 0.25) (layer F.Cu) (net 1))
 (segment (start 142 83.1) (end 141.25 83.1) (width 0.25) (layer F.Cu) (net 1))
 (segment (start 141.25 87.1) (end 142 87.1) (width 0.25) (layer F.Cu) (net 1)) (via (at 158.3 102.8) (size 0.8) (layers F.Cu B.Cu) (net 1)))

